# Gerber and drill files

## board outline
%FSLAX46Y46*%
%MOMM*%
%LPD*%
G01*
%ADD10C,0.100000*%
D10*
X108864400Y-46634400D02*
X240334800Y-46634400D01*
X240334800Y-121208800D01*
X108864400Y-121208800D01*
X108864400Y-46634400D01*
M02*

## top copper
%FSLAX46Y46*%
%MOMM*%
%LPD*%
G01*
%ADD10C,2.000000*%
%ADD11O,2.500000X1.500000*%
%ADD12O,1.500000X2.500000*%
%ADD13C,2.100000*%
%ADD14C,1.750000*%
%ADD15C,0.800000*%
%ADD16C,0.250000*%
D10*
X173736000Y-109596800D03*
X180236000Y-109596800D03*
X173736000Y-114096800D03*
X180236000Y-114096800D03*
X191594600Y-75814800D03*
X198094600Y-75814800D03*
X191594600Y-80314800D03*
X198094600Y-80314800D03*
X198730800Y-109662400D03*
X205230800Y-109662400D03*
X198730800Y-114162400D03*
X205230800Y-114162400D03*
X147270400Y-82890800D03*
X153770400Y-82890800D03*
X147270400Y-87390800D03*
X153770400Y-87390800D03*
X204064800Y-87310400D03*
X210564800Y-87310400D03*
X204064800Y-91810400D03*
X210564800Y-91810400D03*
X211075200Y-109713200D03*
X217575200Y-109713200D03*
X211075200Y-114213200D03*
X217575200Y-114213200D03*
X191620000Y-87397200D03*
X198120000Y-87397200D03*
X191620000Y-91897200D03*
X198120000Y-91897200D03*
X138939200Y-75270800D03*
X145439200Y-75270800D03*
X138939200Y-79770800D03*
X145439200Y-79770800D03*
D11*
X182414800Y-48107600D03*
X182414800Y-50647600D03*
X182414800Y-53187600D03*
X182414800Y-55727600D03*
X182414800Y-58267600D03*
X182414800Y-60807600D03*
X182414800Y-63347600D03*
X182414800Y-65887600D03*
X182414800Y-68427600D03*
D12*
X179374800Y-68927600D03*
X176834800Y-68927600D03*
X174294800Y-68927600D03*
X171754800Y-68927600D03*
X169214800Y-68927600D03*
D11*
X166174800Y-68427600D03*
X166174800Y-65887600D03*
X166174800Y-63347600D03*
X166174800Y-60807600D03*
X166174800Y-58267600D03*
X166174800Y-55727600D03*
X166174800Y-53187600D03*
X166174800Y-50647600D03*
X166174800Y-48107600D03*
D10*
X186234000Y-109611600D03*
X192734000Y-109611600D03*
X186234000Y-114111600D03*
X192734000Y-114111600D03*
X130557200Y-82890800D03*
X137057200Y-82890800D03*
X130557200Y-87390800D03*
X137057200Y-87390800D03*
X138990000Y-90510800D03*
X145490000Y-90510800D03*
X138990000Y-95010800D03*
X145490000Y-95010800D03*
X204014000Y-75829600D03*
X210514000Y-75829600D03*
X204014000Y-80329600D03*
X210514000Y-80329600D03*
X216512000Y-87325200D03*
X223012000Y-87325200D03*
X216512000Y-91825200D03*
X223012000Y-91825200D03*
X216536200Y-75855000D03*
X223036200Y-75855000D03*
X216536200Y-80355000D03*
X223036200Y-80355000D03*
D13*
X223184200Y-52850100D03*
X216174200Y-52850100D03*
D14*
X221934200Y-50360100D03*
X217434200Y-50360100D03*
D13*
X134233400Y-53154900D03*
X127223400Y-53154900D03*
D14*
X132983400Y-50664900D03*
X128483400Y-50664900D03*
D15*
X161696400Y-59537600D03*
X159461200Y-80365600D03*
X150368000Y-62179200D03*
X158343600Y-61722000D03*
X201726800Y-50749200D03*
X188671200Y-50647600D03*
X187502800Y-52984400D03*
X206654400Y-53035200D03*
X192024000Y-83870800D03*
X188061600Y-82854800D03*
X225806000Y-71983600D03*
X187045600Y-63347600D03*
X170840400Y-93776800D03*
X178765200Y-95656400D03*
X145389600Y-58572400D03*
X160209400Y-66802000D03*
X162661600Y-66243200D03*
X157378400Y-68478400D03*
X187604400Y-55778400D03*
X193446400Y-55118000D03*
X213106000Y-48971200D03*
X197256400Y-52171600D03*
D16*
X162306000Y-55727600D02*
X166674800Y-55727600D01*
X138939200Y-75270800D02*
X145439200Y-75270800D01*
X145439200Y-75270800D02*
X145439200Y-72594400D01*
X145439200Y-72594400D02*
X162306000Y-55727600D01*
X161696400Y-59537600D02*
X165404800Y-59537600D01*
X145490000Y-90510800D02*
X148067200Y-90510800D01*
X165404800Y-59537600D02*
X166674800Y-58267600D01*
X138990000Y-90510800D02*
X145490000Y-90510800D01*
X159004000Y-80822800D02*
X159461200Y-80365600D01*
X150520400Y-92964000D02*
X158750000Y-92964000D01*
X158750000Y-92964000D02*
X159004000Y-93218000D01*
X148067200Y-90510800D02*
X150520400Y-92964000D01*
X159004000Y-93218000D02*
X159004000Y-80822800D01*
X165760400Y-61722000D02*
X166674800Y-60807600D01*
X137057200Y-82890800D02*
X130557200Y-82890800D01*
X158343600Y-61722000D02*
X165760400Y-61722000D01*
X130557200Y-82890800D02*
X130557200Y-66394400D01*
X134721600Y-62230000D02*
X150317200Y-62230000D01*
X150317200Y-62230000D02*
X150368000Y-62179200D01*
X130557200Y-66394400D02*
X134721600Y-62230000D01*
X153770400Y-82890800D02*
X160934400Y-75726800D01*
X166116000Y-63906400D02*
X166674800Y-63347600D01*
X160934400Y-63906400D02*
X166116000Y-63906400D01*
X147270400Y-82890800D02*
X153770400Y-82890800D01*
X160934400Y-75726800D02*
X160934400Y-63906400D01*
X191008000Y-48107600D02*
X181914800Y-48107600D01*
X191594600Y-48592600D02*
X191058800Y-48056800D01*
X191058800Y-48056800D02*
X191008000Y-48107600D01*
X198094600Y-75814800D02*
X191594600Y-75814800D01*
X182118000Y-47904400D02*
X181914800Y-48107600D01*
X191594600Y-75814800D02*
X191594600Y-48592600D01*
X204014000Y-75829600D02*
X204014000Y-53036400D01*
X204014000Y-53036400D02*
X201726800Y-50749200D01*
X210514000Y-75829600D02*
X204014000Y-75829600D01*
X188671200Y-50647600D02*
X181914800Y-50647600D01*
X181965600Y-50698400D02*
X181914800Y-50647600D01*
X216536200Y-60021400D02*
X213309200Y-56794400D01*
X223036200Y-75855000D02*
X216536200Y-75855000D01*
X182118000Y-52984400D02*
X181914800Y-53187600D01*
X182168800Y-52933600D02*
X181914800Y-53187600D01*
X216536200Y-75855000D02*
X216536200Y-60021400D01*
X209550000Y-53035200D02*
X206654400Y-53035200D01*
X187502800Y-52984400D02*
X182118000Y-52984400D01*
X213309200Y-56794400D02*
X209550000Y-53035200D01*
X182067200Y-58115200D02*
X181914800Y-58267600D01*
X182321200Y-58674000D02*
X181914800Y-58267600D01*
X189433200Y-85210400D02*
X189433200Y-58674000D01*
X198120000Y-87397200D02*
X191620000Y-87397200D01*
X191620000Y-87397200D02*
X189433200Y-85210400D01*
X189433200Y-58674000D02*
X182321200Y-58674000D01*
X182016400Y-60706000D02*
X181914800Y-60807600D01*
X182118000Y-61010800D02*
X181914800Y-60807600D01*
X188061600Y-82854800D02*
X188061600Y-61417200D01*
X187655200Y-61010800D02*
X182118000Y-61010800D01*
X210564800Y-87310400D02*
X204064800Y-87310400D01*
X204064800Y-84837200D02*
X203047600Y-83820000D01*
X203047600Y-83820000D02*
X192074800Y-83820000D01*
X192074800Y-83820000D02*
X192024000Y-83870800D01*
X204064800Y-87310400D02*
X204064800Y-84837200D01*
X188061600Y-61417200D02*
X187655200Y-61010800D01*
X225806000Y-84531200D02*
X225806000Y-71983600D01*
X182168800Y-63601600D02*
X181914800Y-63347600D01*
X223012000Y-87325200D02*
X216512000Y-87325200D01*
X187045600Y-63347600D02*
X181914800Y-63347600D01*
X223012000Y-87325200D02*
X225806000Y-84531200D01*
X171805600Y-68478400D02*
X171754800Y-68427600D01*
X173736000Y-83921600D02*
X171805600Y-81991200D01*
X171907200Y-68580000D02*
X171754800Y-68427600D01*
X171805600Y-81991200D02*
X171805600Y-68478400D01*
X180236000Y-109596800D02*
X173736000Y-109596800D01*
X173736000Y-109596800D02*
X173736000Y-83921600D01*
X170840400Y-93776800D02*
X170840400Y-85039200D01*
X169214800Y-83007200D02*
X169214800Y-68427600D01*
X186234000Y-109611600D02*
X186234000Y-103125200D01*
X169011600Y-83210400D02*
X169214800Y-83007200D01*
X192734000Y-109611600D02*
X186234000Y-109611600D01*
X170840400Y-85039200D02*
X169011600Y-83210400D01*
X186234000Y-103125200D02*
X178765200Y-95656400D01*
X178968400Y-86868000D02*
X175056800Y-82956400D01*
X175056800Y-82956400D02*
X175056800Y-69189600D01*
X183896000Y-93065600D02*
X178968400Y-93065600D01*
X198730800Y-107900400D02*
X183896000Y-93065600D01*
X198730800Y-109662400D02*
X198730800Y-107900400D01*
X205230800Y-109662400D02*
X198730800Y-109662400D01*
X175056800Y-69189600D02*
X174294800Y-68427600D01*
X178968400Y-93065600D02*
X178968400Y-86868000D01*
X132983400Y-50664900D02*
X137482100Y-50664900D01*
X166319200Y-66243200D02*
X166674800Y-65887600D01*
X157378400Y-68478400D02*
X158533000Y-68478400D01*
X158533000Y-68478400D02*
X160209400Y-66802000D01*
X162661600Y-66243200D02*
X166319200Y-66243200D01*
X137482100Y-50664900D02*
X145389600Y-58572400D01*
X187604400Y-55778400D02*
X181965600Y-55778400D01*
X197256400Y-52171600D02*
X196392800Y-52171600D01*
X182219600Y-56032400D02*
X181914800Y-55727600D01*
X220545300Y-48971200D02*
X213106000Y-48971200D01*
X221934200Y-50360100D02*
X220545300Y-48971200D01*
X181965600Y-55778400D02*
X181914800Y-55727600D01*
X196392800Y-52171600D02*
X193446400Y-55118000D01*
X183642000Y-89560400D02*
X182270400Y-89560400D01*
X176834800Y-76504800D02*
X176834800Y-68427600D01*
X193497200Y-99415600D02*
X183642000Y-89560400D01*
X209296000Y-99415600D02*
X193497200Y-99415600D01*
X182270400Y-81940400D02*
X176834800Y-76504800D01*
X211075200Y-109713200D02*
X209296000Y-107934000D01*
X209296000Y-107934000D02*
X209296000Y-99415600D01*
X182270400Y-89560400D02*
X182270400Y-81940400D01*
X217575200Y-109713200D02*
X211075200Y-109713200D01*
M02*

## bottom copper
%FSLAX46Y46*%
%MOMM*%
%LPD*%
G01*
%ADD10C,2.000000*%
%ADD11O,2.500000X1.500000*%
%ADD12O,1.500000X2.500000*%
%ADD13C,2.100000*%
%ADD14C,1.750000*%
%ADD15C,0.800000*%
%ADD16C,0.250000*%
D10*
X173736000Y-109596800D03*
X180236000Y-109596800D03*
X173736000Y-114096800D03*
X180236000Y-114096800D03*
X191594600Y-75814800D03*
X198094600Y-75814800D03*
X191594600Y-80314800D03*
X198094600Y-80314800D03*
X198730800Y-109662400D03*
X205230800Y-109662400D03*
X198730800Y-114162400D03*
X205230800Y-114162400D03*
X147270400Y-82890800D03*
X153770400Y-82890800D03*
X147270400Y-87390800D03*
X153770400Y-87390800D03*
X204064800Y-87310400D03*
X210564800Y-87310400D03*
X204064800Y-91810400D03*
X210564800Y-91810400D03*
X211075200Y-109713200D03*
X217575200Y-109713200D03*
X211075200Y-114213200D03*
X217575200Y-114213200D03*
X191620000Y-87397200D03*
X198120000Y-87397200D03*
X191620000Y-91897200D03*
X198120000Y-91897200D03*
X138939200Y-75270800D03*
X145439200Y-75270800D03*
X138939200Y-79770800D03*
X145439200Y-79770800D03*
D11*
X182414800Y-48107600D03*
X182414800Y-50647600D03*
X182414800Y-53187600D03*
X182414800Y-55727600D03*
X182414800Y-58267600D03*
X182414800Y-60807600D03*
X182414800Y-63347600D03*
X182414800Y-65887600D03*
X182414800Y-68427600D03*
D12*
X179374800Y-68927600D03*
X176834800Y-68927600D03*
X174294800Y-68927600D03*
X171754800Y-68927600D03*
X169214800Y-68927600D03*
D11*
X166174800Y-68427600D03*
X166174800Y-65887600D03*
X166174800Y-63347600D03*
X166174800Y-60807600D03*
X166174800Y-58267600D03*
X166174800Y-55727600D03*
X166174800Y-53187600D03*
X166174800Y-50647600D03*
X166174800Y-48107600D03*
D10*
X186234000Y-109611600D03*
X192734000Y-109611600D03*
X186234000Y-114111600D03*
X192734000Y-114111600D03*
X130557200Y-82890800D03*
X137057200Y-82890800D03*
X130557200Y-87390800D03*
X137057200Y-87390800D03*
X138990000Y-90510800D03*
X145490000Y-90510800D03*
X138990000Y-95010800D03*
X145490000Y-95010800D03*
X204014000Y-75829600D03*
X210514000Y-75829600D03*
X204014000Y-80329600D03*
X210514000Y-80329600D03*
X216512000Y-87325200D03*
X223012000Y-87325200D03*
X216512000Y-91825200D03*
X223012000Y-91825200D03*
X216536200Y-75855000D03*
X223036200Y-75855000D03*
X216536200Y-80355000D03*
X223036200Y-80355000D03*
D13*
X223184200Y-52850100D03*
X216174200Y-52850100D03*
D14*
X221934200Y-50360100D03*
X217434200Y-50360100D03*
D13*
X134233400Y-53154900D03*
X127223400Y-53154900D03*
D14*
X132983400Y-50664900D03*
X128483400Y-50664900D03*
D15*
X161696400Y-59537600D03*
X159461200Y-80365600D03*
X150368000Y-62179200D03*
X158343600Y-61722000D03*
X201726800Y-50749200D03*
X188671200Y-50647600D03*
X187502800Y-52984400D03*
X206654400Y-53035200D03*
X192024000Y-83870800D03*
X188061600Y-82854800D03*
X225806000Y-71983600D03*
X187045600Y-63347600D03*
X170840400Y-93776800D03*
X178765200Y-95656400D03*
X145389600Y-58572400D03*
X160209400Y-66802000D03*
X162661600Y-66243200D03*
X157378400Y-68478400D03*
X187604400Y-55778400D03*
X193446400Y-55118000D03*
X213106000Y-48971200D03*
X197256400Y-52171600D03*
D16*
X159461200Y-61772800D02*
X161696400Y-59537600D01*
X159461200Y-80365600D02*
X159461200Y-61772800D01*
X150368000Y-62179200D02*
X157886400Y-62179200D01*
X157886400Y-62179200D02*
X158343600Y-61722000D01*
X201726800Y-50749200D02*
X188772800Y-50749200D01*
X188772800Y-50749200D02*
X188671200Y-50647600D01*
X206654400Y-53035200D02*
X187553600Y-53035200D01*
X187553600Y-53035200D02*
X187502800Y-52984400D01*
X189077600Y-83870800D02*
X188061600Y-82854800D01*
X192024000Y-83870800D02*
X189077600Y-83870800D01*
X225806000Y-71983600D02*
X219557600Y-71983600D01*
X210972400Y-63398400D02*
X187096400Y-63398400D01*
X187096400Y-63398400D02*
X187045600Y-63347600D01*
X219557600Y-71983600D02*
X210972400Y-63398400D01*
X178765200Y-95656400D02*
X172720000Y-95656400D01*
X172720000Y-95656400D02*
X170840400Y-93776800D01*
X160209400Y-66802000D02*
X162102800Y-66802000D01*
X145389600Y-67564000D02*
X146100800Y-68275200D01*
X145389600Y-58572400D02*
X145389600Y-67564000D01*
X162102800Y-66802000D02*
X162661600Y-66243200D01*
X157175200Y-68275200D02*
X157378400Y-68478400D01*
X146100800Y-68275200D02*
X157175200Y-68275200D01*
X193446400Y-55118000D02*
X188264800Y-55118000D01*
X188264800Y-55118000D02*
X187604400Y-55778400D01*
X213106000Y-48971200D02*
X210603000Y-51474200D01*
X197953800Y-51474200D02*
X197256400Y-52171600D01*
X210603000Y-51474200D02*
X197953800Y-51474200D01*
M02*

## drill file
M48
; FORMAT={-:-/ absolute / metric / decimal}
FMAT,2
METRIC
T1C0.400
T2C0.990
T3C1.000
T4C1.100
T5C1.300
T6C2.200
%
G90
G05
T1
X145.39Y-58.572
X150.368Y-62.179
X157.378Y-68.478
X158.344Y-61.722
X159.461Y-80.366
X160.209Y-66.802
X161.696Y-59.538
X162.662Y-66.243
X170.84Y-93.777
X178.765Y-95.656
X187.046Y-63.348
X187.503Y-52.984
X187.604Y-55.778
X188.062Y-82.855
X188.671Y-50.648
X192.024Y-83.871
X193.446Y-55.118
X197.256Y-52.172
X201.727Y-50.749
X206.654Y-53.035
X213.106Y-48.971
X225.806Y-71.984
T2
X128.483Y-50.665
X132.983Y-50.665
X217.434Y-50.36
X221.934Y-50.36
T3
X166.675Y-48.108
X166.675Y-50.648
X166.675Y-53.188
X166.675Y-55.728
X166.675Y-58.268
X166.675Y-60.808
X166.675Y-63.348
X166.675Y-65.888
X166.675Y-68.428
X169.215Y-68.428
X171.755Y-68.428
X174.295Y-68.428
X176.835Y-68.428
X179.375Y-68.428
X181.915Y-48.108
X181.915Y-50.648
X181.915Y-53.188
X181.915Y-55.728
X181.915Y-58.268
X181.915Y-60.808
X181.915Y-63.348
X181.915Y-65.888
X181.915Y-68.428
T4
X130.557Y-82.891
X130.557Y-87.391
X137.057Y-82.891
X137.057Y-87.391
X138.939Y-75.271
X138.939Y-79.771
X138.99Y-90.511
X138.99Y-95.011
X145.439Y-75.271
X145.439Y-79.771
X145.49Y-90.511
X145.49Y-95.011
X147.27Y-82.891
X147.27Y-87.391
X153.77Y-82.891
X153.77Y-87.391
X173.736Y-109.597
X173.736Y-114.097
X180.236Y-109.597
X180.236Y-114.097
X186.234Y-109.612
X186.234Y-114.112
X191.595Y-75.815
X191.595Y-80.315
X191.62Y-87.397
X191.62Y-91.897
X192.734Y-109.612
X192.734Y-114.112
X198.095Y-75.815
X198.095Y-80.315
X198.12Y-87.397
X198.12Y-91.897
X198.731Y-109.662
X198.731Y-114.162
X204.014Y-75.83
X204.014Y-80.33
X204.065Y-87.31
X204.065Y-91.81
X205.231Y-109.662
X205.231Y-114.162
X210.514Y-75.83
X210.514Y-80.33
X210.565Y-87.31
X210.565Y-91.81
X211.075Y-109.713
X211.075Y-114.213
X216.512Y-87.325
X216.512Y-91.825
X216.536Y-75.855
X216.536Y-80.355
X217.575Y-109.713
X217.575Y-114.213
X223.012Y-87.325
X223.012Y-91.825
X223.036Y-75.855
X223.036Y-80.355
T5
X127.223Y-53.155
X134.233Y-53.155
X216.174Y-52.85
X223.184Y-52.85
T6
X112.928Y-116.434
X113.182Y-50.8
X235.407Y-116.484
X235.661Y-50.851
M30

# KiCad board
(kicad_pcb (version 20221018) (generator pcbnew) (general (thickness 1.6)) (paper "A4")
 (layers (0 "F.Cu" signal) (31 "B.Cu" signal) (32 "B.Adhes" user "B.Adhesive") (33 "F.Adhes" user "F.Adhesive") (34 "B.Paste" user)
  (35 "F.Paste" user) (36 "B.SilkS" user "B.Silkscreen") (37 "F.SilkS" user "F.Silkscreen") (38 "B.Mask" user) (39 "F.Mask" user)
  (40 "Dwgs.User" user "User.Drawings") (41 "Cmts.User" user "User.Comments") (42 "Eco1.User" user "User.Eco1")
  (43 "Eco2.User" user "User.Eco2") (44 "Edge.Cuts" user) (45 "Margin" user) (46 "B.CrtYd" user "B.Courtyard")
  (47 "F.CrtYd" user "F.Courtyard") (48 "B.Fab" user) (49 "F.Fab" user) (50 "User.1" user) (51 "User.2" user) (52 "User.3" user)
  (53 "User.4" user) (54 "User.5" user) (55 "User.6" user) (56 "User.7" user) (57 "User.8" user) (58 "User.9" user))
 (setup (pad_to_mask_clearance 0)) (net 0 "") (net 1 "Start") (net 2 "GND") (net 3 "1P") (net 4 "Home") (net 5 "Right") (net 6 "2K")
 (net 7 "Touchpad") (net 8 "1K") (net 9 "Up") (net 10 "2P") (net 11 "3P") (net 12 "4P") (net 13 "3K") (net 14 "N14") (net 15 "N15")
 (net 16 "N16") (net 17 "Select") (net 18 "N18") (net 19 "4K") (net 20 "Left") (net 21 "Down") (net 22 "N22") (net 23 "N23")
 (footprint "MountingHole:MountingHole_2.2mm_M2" (layer "F.Cu") (at 112.9284 116.4336)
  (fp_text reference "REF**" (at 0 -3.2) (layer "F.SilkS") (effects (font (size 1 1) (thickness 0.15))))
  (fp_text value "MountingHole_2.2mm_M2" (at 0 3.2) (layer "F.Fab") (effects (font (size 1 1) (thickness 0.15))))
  (pad "" np_thru_hole circle (at 0 0) (size 2.2 2.2) (drill 2.2) (layers "F&B.Cu" "*.Mask")))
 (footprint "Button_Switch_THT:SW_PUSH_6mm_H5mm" (layer "F.Cu") (at 173.736 109.5968)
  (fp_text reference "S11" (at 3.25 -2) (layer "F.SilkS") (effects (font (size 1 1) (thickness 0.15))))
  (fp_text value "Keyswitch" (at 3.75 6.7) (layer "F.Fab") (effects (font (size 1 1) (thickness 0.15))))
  (pad "1" thru_hole circle (at 0 0 90) (size 2 2) (drill 1.1) (layers "*.Cu" "*.Mask") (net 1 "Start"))
  (pad "1" thru_hole circle (at 6.5 0 90) (size 2 2) (drill 1.1) (layers "*.Cu" "*.Mask") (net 1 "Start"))
  (pad "2" thru_hole circle (at 0 4.5 90) (size 2 2) (drill 1.1) (layers "*.Cu" "*.Mask") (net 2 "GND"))
  (pad "2" thru_hole circle (at 6.5 4.5 90) (size 2 2) (drill 1.1) (layers "*.Cu" "*.Mask") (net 2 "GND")))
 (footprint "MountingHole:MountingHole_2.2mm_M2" (layer "F.Cu") (at 113.1824 50.8)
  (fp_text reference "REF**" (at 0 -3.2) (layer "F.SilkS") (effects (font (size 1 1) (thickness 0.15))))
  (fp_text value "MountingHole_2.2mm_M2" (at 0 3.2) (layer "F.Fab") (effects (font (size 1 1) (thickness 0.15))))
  (pad "" np_thru_hole circle (at 0 0) (size 2.2 2.2) (drill 2.2) (layers "F&B.Cu" "*.Mask")))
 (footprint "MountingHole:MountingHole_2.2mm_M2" (layer "F.Cu") (at 235.4072 116.4844)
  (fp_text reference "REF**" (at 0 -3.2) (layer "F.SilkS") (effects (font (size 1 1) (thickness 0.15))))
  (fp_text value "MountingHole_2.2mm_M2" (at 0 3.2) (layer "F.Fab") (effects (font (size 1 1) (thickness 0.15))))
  (pad "" np_thru_hole circle (at 0 0) (size 2.2 2.2) (drill 2.2) (layers "F&B.Cu" "*.Mask")))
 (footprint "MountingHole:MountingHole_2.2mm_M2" (layer "F.Cu") (at 235.6612 50.8508)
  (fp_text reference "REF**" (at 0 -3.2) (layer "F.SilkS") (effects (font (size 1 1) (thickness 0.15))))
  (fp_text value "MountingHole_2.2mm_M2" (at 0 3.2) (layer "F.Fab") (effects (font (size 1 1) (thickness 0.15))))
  (pad "" np_thru_hole circle (at 0 0) (size 2.2 2.2) (drill 2.2) (layers "*.Cu" "*.Mask")))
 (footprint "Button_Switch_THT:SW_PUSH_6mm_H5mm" (layer "F.Cu") (at 191.5946 75.8148)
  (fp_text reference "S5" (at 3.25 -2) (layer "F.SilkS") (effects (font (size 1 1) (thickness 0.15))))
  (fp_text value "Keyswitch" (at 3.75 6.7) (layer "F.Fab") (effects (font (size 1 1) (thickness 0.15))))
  (pad "1" thru_hole circle (at 0 0 90) (size 2 2) (drill 1.1) (layers "*.Cu" "*.Mask") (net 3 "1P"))
  (pad "1" thru_hole circle (at 6.5 0 90) (size 2 2) (drill 1.1) (layers "*.Cu" "*.Mask") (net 3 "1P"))
  (pad "2" thru_hole circle (at 0 4.5 90) (size 2 2) (drill 1.1) (layers "*.Cu" "*.Mask") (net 2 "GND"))
  (pad "2" thru_hole circle (at 6.5 4.5 90) (size 2 2) (drill 1.1) (layers "*.Cu" "*.Mask") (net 2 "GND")))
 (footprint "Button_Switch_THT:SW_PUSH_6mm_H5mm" (layer "F.Cu") (at 198.7308 109.6624)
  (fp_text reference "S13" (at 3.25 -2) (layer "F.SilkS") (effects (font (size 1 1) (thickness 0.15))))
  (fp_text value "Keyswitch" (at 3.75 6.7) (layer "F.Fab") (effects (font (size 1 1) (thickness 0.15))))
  (pad "1" thru_hole circle (at 0 0 90) (size 2 2) (drill 1.1) (layers "*.Cu" "*.Mask") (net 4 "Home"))
  (pad "1" thru_hole circle (at 6.5 0 90) (size 2 2) (drill 1.1) (layers "*.Cu" "*.Mask") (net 4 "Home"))
  (pad "2" thru_hole circle (at 0 4.5 90) (size 2 2) (drill 1.1) (layers "*.Cu" "*.Mask") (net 2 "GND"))
  (pad "2" thru_hole circle (at 6.5 4.5 90) (size 2 2) (drill 1.1) (layers "*.Cu" "*.Mask") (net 2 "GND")))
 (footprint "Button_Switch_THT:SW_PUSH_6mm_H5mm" (layer "F.Cu") (at 147.2704 82.8908)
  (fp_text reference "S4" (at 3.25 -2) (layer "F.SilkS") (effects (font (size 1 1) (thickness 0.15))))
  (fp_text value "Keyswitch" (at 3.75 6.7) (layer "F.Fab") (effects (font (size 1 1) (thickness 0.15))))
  (pad "1" thru_hole circle (at 0 0 90) (size 2 2) (drill 1.1) (layers "*.Cu" "*.Mask") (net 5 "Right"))
  (pad "1" thru_hole circle (at 6.5 0 90) (size 2 2) (drill 1.1) (layers "*.Cu" "*.Mask") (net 5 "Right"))
  (pad "2" thru_hole circle (at 0 4.5 90) (size 2 2) (drill 1.1) (layers "*.Cu" "*.Mask") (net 2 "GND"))
  (pad "2" thru_hole circle (at 6.5 4.5 90) (size 2 2) (drill 1.1) (layers "*.Cu" "*.Mask") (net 2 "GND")))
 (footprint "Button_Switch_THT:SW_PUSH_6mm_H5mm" (layer "F.Cu") (at 204.0648 87.3104)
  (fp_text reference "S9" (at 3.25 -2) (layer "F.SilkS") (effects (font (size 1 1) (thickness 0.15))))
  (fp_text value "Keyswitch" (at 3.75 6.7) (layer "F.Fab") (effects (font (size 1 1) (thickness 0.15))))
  (pad "1" thru_hole circle (at 0 0 90) (size 2 2) (drill 1.1) (layers "*.Cu" "*.Mask") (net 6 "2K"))
  (pad "1" thru_hole circle (at 6.5 0 90) (size 2 2) (drill 1.1) (layers "*.Cu" "*.Mask") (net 6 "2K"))
  (pad "2" thru_hole circle (at 0 4.5 90) (size 2 2) (drill 1.1) (layers "*.Cu" "*.Mask") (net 2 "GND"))
  (pad "2" thru_hole circle (at 6.5 4.5 90) (size 2 2) (drill 1.1) (layers "*.Cu" "*.Mask") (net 2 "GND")))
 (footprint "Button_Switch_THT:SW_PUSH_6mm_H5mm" (layer "F.Cu") (at 211.0752 109.7132)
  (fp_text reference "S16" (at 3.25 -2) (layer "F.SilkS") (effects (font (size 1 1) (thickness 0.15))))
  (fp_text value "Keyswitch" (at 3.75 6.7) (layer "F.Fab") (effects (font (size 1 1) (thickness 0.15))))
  (pad "1" thru_hole circle (at 0 0 90) (size 2 2) (drill 1.1) (layers "*.Cu" "*.Mask") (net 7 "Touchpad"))
  (pad "1" thru_hole circle (at 6.5 0 90) (size 2 2) (drill 1.1) (layers "*.Cu" "*.Mask") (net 7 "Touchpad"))
  (pad "2" thru_hole circle (at 0 4.5 90) (size 2 2) (drill 1.1) (layers "*.Cu" "*.Mask") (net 2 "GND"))
  (pad "2" thru_hole circle (at 6.5 4.5 90) (size 2 2) (drill 1.1) (layers "*.Cu" "*.Mask") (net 2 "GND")))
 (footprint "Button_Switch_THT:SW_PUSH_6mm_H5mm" (layer "F.Cu") (at 191.62 87.3972)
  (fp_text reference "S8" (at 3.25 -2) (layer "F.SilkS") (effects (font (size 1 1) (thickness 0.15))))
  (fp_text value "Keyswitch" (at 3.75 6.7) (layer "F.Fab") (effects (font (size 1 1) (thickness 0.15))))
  (pad "1" thru_hole circle (at 0 0 90) (size 2 2) (drill 1.1) (layers "*.Cu" "*.Mask") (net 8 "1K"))
  (pad "1" thru_hole circle (at 6.5 0 90) (size 2 2) (drill 1.1) (layers "*.Cu" "*.Mask") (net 8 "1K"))
  (pad "2" thru_hole circle (at 0 4.5 90) (size 2 2) (drill 1.1) (layers "*.Cu" "*.Mask") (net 2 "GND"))
  (pad "2" thru_hole circle (at 6.5 4.5 90) (size 2 2) (drill 1.1) (layers "*.Cu" "*.Mask") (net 2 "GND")))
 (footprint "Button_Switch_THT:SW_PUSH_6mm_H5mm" (layer "F.Cu") (at 138.9392 75.2708)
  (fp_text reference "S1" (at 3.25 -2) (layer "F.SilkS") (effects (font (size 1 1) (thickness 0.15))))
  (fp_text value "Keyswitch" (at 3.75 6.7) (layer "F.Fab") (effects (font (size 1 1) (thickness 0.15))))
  (pad "1" thru_hole circle (at 0 0 90) (size 2 2) (drill 1.1) (layers "*.Cu" "*.Mask") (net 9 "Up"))
  (pad "1" thru_hole circle (at 6.5 0 90) (size 2 2) (drill 1.1) (layers "*.Cu" "*.Mask") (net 9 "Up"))
  (pad "2" thru_hole circle (at 0 4.5 90) (size 2 2) (drill 1.1) (layers "*.Cu" "*.Mask") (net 2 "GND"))
  (pad "2" thru_hole circle (at 6.5 4.5 90) (size 2 2) (drill 1.1) (layers "*.Cu" "*.Mask") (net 2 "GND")))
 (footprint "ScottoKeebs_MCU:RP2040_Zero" (layer "F.Cu") (at 174.2948 58.2676)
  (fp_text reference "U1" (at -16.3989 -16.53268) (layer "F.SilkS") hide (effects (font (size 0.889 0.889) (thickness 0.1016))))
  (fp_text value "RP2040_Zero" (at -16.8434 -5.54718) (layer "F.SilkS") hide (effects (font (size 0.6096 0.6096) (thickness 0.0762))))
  (pad "1" thru_hole oval (at 7.62 -10.16 180) (size 2.5 1.5) (drill 1 (offset -0.5 0)) (layers "*.Cu" "*.Mask") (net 3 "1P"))
  (pad "2" thru_hole oval (at 7.62 -7.62 180) (size 2.5 1.5) (drill 1 (offset -0.5 0)) (layers "*.Cu" "*.Mask") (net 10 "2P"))
  (pad "3" thru_hole oval (at 7.62 -5.08 180) (size 2.5 1.5) (drill 1 (offset -0.5 0)) (layers "*.Cu" "*.Mask") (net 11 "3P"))
  (pad "4" thru_hole oval (at 7.62 -2.54 180) (size 2.5 1.5) (drill 1 (offset -0.5 0)) (layers "*.Cu" "*.Mask") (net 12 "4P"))
  (pad "5" thru_hole oval (at 7.62 0 180) (size 2.5 1.5) (drill 1 (offset -0.5 0)) (layers "*.Cu" "*.Mask") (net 8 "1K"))
  (pad "6" thru_hole oval (at 7.62 2.54 180) (size 2.5 1.5) (drill 1 (offset -0.5 0)) (layers "*.Cu" "*.Mask") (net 6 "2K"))
  (pad "7" thru_hole oval (at 7.62 5.08 180) (size 2.5 1.5) (drill 1 (offset -0.5 0)) (layers "*.Cu" "*.Mask") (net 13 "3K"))
  (pad "8" thru_hole oval (at 7.62 7.62 180) (size 2.5 1.5) (drill 1 (offset -0.5 0)) (layers "*.Cu" "*.Mask") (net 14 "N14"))
  (pad "9" thru_hole oval (at 7.62 10.16 180) (size 2.5 1.5) (drill 1 (offset -0.5 0)) (layers "*.Cu" "*.Mask") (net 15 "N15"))
  (pad "10" thru_hole oval (at 5.08 10.16 90) (size 2.5 1.5) (drill 1 (offset -0.5 0)) (layers "*.Cu" "*.Mask") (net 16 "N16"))
  (pad "11" thru_hole oval (at 2.54 10.16 90) (size 2.5 1.5) (drill 1 (offset -0.5 0)) (layers "*.Cu" "*.Mask") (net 7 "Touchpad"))
  (pad "12" thru_hole oval (at 0 10.16 90) (size 2.5 1.5) (drill 1 (offset -0.5 0)) (layers "*.Cu" "*.Mask") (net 4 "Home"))
  (pad "13" thru_hole oval (at -2.54 10.16 90) (size 2.5 1.5) (drill 1 (offset -0.5 0)) (layers "*.Cu" "*.Mask") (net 1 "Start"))
  (pad "14" thru_hole oval (at -5.08 10.16 90) (size 2.5 1.5) (drill 1 (offset -0.5 0)) (layers "*.Cu" "*.Mask") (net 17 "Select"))
  (pad "15" thru_hole oval (at -7.62 10.16) (size 2.5 1.5) (drill 1 (offset -0.5 0)) (layers "*.Cu" "*.Mask") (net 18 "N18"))
  (pad "16" thru_hole oval (at -7.62 7.62) (size 2.5 1.5) (drill 1 (offset -0.5 0)) (layers "*.Cu" "*.Mask") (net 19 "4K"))
  (pad "17" thru_hole oval (at -7.62 5.08) (size 2.5 1.5) (drill 1 (offset -0.5 0)) (layers "*.Cu" "*.Mask") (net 5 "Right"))
  (pad "18" thru_hole oval (at -7.62 2.54) (size 2.5 1.5) (drill 1 (offset -0.5 0)) (layers "*.Cu" "*.Mask") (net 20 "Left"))
  (pad "19" thru_hole oval (at -7.62 0) (size 2.5 1.5) (drill 1 (offset -0.5 0)) (layers "*.Cu" "*.Mask") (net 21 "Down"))
  (pad "20" thru_hole oval (at -7.62 -2.54) (size 2.5 1.5) (drill 1 (offset -0.5 0)) (layers "*.Cu" "*.Mask") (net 9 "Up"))
  (pad "21" thru_hole oval (at -7.62 -5.08) (size 2.5 1.5) (drill 1 (offset -0.5 0)) (layers "*.Cu" "*.Mask") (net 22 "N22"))
  (pad "22" thru_hole oval (at -7.62 -7.62) (size 2.5 1.5) (drill 1 (offset -0.5 0)) (layers "*.Cu" "*.Mask") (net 2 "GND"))
  (pad "23" thru_hole oval (at -7.62 -10.16) (size 2.5 1.5) (drill 1 (offset -0.5 0)) (layers "*.Cu" "*.Mask") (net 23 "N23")))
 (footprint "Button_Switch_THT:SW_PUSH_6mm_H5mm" (layer "F.Cu") (at 186.234 109.6116)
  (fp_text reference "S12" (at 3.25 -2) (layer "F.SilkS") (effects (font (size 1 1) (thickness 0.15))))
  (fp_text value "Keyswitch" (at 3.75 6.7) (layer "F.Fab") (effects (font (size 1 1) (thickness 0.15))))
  (pad "1" thru_hole circle (at 0 0 90) (size 2 2) (drill 1.1) (layers "*.Cu" "*.Mask") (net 17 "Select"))
  (pad "1" thru_hole circle (at 6.5 0 90) (size 2 2) (drill 1.1) (layers "*.Cu" "*.Mask") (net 17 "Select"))
  (pad "2" thru_hole circle (at 0 4.5 90) (size 2 2) (drill 1.1) (layers "*.Cu" "*.Mask") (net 2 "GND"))
  (pad "2" thru_hole circle (at 6.5 4.5 90) (size 2 2) (drill 1.1) (layers "*.Cu" "*.Mask") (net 2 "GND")))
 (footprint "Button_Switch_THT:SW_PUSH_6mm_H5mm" (layer "F.Cu") (at 130.5572 82.8908)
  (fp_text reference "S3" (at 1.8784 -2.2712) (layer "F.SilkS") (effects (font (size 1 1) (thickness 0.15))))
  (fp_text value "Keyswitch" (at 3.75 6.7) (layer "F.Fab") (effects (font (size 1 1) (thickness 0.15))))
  (pad "1" thru_hole circle (at 0 0 90) (size 2 2) (drill 1.1) (layers "*.Cu" "*.Mask") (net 20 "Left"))
  (pad "1" thru_hole circle (at 6.5 0 90) (size 2 2) (drill 1.1) (layers "*.Cu" "*.Mask") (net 20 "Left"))
  (pad "2" thru_hole circle (at 0 4.5 90) (size 2 2) (drill 1.1) (layers "*.Cu" "*.Mask") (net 2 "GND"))
  (pad "2" thru_hole circle (at 6.5 4.5 90) (size 2 2) (drill 1.1) (layers "*.Cu" "*.Mask") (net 2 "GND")))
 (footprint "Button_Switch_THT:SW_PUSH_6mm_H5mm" (layer "F.Cu") (at 138.99 90.5108)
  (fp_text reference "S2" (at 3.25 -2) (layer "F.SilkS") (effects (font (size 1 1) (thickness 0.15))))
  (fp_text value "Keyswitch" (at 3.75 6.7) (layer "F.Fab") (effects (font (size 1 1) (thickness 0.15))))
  (pad "1" thru_hole circle (at 0 0 90) (size 2 2) (drill 1.1) (layers "*.Cu" "*.Mask") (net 21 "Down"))
  (pad "1" thru_hole circle (at 6.5 0 90) (size 2 2) (drill 1.1) (layers "*.Cu" "*.Mask") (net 21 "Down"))
  (pad "2" thru_hole circle (at 0 4.5 90) (size 2 2) (drill 1.1) (layers "*.Cu" "*.Mask") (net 2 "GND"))
  (pad "2" thru_hole circle (at 6.5 4.5 90) (size 2 2) (drill 1.1) (layers "*.Cu" "*.Mask") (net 2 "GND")))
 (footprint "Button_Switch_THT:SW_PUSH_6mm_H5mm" (layer "F.Cu") (at 204.014 75.8296)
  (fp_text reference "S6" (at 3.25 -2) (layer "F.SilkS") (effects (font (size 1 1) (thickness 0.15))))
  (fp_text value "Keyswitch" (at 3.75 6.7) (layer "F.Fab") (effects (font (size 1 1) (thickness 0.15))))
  (pad "1" thru_hole circle (at 0 0 90) (size 2 2) (drill 1.1) (layers "*.Cu" "*.Mask") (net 10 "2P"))
  (pad "1" thru_hole circle (at 6.5 0 90) (size 2 2) (drill 1.1) (layers "*.Cu" "*.Mask") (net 10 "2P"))
  (pad "2" thru_hole circle (at 0 4.5 90) (size 2 2) (drill 1.1) (layers "*.Cu" "*.Mask") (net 2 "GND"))
  (pad "2" thru_hole circle (at 6.5 4.5 90) (size 2 2) (drill 1.1) (layers "*.Cu" "*.Mask") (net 2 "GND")))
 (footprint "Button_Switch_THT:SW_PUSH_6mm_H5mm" (layer "F.Cu") (at 216.512 87.3252)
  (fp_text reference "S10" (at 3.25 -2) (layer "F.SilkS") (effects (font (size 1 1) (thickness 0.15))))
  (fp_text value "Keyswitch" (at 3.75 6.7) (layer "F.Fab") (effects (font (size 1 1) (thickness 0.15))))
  (pad "1" thru_hole circle (at 0 0 90) (size 2 2) (drill 1.1) (layers "*.Cu" "*.Mask") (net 13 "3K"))
  (pad "1" thru_hole circle (at 6.5 0 90) (size 2 2) (drill 1.1) (layers "*.Cu" "*.Mask") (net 13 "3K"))
  (pad "2" thru_hole circle (at 0 4.5 90) (size 2 2) (drill 1.1) (layers "*.Cu" "*.Mask") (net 2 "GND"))
  (pad "2" thru_hole circle (at 6.5 4.5 90) (size 2 2) (drill 1.1) (layers "*.Cu" "*.Mask") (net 2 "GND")))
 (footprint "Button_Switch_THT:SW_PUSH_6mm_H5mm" (layer "F.Cu") (at 216.5362 75.855)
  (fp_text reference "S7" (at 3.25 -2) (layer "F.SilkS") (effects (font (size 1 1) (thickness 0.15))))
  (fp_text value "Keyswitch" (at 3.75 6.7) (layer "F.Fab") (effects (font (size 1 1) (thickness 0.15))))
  (pad "1" thru_hole circle (at 0 0 90) (size 2 2) (drill 1.1) (layers "*.Cu" "*.Mask") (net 11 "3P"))
  (pad "1" thru_hole circle (at 6.5 0 90) (size 2 2) (drill 1.1) (layers "*.Cu" "*.Mask") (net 11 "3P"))
  (pad "2" thru_hole circle (at 0 4.5 90) (size 2 2) (drill 1.1) (layers "*.Cu" "*.Mask") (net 2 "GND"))
  (pad "2" thru_hole circle (at 6.5 4.5 90) (size 2 2) (drill 1.1) (layers "*.Cu" "*.Mask") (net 2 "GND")))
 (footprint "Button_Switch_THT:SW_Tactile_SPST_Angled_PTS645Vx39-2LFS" (layer "B.Cu") (at 221.9342 50.3601 180)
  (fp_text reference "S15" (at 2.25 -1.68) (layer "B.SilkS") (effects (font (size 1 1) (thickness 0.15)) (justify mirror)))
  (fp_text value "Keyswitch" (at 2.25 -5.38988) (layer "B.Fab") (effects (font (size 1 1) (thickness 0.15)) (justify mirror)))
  (pad "" thru_hole circle (at -1.25 -2.49 180) (size 2.1 2.1) (drill 1.3) (layers "*.Cu" "*.Mask"))
  (pad "" thru_hole circle (at 5.76 -2.49 180) (size 2.1 2.1) (drill 1.3) (layers "*.Cu" "*.Mask"))
  (pad "1" thru_hole circle (at 0 0 180) (size 1.75 1.75) (drill 0.99) (layers "*.Cu" "*.Mask") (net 12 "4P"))
  (pad "2" thru_hole circle (at 4.5 0 180) (size 1.75 1.75) (drill 0.99) (layers "*.Cu" "*.Mask") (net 2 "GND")))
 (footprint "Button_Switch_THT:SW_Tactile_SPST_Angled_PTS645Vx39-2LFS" (layer "B.Cu") (at 132.9834 50.6649 180)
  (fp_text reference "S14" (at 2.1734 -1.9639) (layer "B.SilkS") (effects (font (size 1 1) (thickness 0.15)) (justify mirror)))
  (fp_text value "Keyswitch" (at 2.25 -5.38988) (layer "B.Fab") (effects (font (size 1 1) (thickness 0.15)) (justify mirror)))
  (pad "" thru_hole circle (at -1.25 -2.49 180) (size 2.1 2.1) (drill 1.3) (layers "*.Cu" "*.Mask"))
  (pad "" thru_hole circle (at 5.76 -2.49 180) (size 2.1 2.1) (drill 1.3) (layers "*.Cu" "*.Mask"))
  (pad "1" thru_hole circle (at 0 0 180) (size 1.75 1.75) (drill 0.99) (layers "*.Cu" "*.Mask") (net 19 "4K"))
  (pad "2" thru_hole circle (at 4.5 0 180) (size 1.75 1.75) (drill 0.99) (layers "*.Cu" "*.Mask") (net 2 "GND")))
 (gr_rect (start 108.8644 46.6344) (end 240.3348 121.2088) (stroke (width 0.1) (type default)) (fill none) (layer "Edge.Cuts"))
 (segment (start 162.306 55.7276) (end 166.6748 55.7276) (width 0.25) (layer "F.Cu") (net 9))
 (segment (start 138.9392 75.2708) (end 145.4392 75.2708) (width 0.25) (layer "F.Cu") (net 9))
 (segment (start 145.4392 75.2708) (end 145.4392 72.5944) (width 0.25) (layer "F.Cu") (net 9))
 (segment (start 145.4392 72.5944) (end 162.306 55.7276) (width 0.25) (layer "F.Cu") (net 9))
 (segment (start 161.6964 59.5376) (end 165.4048 59.5376) (width 0.25) (layer "F.Cu") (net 21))
 (segment (start 145.49 90.5108) (end 148.0672 90.5108) (width 0.25) (layer "F.Cu") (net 21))
 (segment (start 165.4048 59.5376) (end 166.6748 58.2676) (width 0.25) (layer "F.Cu") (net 21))
 (segment (start 138.99 90.5108) (end 145.49 90.5108) (width 0.25) (layer "F.Cu") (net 21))
 (segment (start 159.004 80.8228) (end 159.4612 80.3656) (width 0.25) (layer "F.Cu") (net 21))
 (segment (start 150.5204 92.964) (end 158.75 92.964) (width 0.25) (layer "F.Cu") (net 21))
 (segment (start 158.75 92.964) (end 159.004 93.218) (width 0.25) (layer "F.Cu") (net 21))
 (segment (start 148.0672 90.5108) (end 150.5204 92.964) (width 0.25) (layer "F.Cu") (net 21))
 (segment (start 159.004 93.218) (end 159.004 80.8228) (width 0.25) (layer "F.Cu") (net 21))
 (via (at 161.6964 59.5376) (size 0.8) (drill 0.4) (layers "F.Cu" "B.Cu") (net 21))
 (via (at 159.4612 80.3656) (size 0.8) (drill 0.4) (layers "F.Cu" "B.Cu") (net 21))
 (segment (start 159.4612 61.7728) (end 161.6964 59.5376) (width 0.25) (layer "B.Cu") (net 21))
 (segment (start 159.4612 80.3656) (end 159.4612 61.7728) (width 0.25) (layer "B.Cu") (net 21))
 (segment (start 165.7604 61.722) (end 166.6748 60.8076) (width 0.25) (layer "F.Cu") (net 20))
 (segment (start 137.0572 82.8908) (end 130.5572 82.8908) (width 0.25) (layer "F.Cu") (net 20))
 (segment (start 158.3436 61.722) (end 165.7604 61.722) (width 0.25) (layer "F.Cu") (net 20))
 (segment (start 130.5572 82.8908) (end 130.5572 66.3944) (width 0.25) (layer "F.Cu") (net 20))
 (segment (start 134.7216 62.23) (end 150.3172 62.23) (width 0.25) (layer "F.Cu") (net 20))
 (segment (start 150.3172 62.23) (end 150.368 62.1792) (width 0.25) (layer "F.Cu") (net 20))
 (segment (start 130.5572 66.3944) (end 134.7216 62.23) (width 0.25) (layer "F.Cu") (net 20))
 (via (at 150.368 62.1792) (size 0.8) (drill 0.4) (layers "F.Cu" "B.Cu") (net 20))
 (via (at 158.3436 61.722) (size 0.8) (drill 0.4) (layers "F.Cu" "B.Cu") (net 20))
 (segment (start 150.368 62.1792) (end 157.8864 62.1792) (width 0.25) (layer "B.Cu") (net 20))
 (segment (start 157.8864 62.1792) (end 158.3436 61.722) (width 0.25) (layer "B.Cu") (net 20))
 (segment (start 153.7704 82.8908) (end 160.9344 75.7268) (width 0.25) (layer "F.Cu") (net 5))
 (segment (start 166.116 63.9064) (end 166.6748 63.3476) (width 0.25) (layer "F.Cu") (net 5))
 (segment (start 160.9344 63.9064) (end 166.116 63.9064) (width 0.25) (layer "F.Cu") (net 5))
 (segment (start 147.2704 82.8908) (end 153.7704 82.8908) (width 0.25) (layer "F.Cu") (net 5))
 (segment (start 160.9344 75.7268) (end 160.9344 63.9064) (width 0.25) (layer "F.Cu") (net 5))
 (segment (start 191.008 48.1076) (end 181.9148 48.1076) (width 0.25) (layer "F.Cu") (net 3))
 (segment (start 191.5946 48.5926) (end 191.0588 48.0568) (width 0.25) (layer "F.Cu") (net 3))
 (segment (start 191.0588 48.0568) (end 191.008 48.1076) (width 0.25) (layer "F.Cu") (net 3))
 (segment (start 198.0946 75.8148) (end 191.5946 75.8148) (width 0.25) (layer "F.Cu") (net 3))
 (segment (start 182.118 47.9044) (end 181.9148 48.1076) (width 0.25) (layer "F.Cu") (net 3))
 (segment (start 191.5946 75.8148) (end 191.5946 48.5926) (width 0.25) (layer "F.Cu") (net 3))
 (segment (start 204.014 75.8296) (end 204.014 53.0364) (width 0.25) (layer "F.Cu") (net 10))
 (segment (start 204.014 53.0364) (end 201.7268 50.7492) (width 0.25) (layer "F.Cu") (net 10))
 (segment (start 210.514 75.8296) (end 204.014 75.8296) (width 0.25) (layer "F.Cu") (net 10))
 (segment (start 188.6712 50.6476) (end 181.9148 50.6476) (width 0.25) (layer "F.Cu") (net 10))
 (segment (start 181.9656 50.6984) (end 181.9148 50.6476) (width 0.25) (layer "F.Cu") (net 10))
 (via (at 201.7268 50.7492) (size 0.8) (drill 0.4) (layers "F.Cu" "B.Cu") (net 10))
 (via (at 188.6712 50.6476) (size 0.8) (drill 0.4) (layers "F.Cu" "B.Cu") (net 10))
 (segment (start 201.7268 50.7492) (end 188.7728 50.7492) (width 0.25) (layer "B.Cu") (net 10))
 (segment (start 188.7728 50.7492) (end 188.6712 50.6476) (width 0.25) (layer "B.Cu") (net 10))
 (segment (start 216.5362 60.0214) (end 213.3092 56.7944) (width 0.25) (layer "F.Cu") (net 11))
 (segment (start 223.0362 75.855) (end 216.5362 75.855) (width 0.25) (layer "F.Cu") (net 11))
 (segment (start 182.118 52.9844) (end 181.9148 53.1876) (width 0.25) (layer "F.Cu") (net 11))
 (segment (start 182.1688 52.9336) (end 181.9148 53.1876) (width 0.25) (layer "F.Cu") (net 11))
 (segment (start 216.5362 75.855) (end 216.5362 60.0214) (width 0.25) (layer "F.Cu") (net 11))
 (segment (start 209.55 53.0352) (end 206.6544 53.0352) (width 0.25) (layer "F.Cu") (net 11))
 (segment (start 187.5028 52.9844) (end 182.118 52.9844) (width 0.25) (layer "F.Cu") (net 11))
 (segment (start 213.3092 56.7944) (end 209.55 53.0352) (width 0.25) (layer "F.Cu") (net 11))
 (via (at 187.5028 52.9844) (size 0.8) (drill 0.4) (layers "F.Cu" "B.Cu") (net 11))
 (via (at 206.6544 53.0352) (size 0.8) (drill 0.4) (layers "F.Cu" "B.Cu") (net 11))
 (segment (start 206.6544 53.0352) (end 187.5536 53.0352) (width 0.25) (layer "B.Cu") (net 11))
 (segment (start 187.5536 53.0352) (end 187.5028 52.9844) (width 0.25) (layer "B.Cu") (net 11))
 (segment (start 182.0672 58.1152) (end 181.9148 58.2676) (width 0.25) (layer "F.Cu") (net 8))
 (segment (start 182.3212 58.674) (end 181.9148 58.2676) (width 0.25) (layer "F.Cu") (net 8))
 (segment (start 189.4332 85.2104) (end 189.4332 58.674) (width 0.25) (layer "F.Cu") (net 8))
 (segment (start 198.12 87.3972) (end 191.62 87.3972) (width 0.25) (layer "F.Cu") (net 8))
 (segment (start 191.62 87.3972) (end 189.4332 85.2104) (width 0.25) (layer "F.Cu") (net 8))
 (segment (start 189.4332 58.674) (end 182.3212 58.674) (width 0.25) (layer "F.Cu") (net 8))
 (segment (start 182.0164 60.706) (end 181.9148 60.8076) (width 0.25) (layer "F.Cu") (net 6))
 (segment (start 182.118 61.0108) (end 181.9148 60.8076) (width 0.25) (layer "F.Cu") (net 6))
 (segment (start 188.0616 82.8548) (end 188.0616 61.4172) (width 0.25) (layer "F.Cu") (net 6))
 (segment (start 187.6552 61.0108) (end 182.118 61.0108) (width 0.25) (layer "F.Cu") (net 6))
 (segment (start 210.5648 87.3104) (end 204.0648 87.3104) (width 0.25) (layer "F.Cu") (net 6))
 (segment (start 204.0648 84.8372) (end 203.0476 83.82) (width 0.25) (layer "F.Cu") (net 6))
 (segment (start 203.0476 83.82) (end 192.0748 83.82) (width 0.25) (layer "F.Cu") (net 6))
 (segment (start 192.0748 83.82) (end 192.024 83.8708) (width 0.25) (layer "F.Cu") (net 6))
 (segment (start 204.0648 87.3104) (end 204.0648 84.8372) (width 0.25) (layer "F.Cu") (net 6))
 (segment (start 188.0616 61.4172) (end 187.6552 61.0108) (width 0.25) (layer "F.Cu") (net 6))
 (via (at 192.024 83.8708) (size 0.8) (drill 0.4) (layers "F.Cu" "B.Cu") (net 6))
 (via (at 188.0616 82.8548) (size 0.8) (drill 0.4) (layers "F.Cu" "B.Cu") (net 6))
 (segment (start 189.0776 83.8708) (end 188.0616 82.8548) (width 0.25) (layer "B.Cu") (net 6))
 (segment (start 192.024 83.8708) (end 189.0776 83.8708) (width 0.25) (layer "B.Cu") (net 6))
 (segment (start 225.806 84.5312) (end 225.806 71.9836) (width 0.25) (layer "F.Cu") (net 13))
 (segment (start 182.1688 63.6016) (end 181.9148 63.3476) (width 0.25) (layer "F.Cu") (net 13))
 (segment (start 223.012 87.3252) (end 216.512 87.3252) (width 0.25) (layer "F.Cu") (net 13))
 (segment (start 187.0456 63.3476) (end 181.9148 63.3476) (width 0.25) (layer "F.Cu") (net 13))
 (segment (start 223.012 87.3252) (end 225.806 84.5312) (width 0.25) (layer "F.Cu") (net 13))
 (via (at 225.806 71.9836) (size 0.8) (drill 0.4) (layers "F.Cu" "B.Cu") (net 13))
 (via (at 187.0456 63.3476) (size 0.8) (drill 0.4) (layers "F.Cu" "B.Cu") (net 13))
 (segment (start 225.806 71.9836) (end 219.5576 71.9836) (width 0.25) (layer "B.Cu") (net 13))
 (segment (start 210.9724 63.3984) (end 187.0964 63.3984) (width 0.25) (layer "B.Cu") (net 13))
 (segment (start 187.0964 63.3984) (end 187.0456 63.3476) (width 0.25) (layer "B.Cu") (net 13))
 (segment (start 219.5576 71.9836) (end 210.9724 63.3984) (width 0.25) (layer "B.Cu") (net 13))
 (segment (start 171.8056 68.4784) (end 171.7548 68.4276) (width 0.25) (layer "F.Cu") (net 1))
 (segment (start 173.736 83.9216) (end 171.8056 81.9912) (width 0.25) (layer "F.Cu") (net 1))
 (segment (start 171.9072 68.58) (end 171.7548 68.4276) (width 0.25) (layer "F.Cu") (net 1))
 (segment (start 171.8056 81.9912) (end 171.8056 68.4784) (width 0.25) (layer "F.Cu") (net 1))
 (segment (start 180.236 109.5968) (end 173.736 109.5968) (width 0.25) (layer "F.Cu") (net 1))
 (segment (start 173.736 109.5968) (end 173.736 83.9216) (width 0.25) (layer "F.Cu") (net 1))
 (segment (start 170.8404 93.7768) (end 170.8404 85.0392) (width 0.25) (layer "F.Cu") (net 17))
 (segment (start 169.2148 83.0072) (end 169.2148 68.4276) (width 0.25) (layer "F.Cu") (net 17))
 (segment (start 186.234 109.6116) (end 186.234 103.1252) (width 0.25) (layer "F.Cu") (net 17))
 (segment (start 169.0116 83.2104) (end 169.2148 83.0072) (width 0.25) (layer "F.Cu") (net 17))
 (segment (start 192.734 109.6116) (end 186.234 109.6116) (width 0.25) (layer "F.Cu") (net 17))
 (segment (start 170.8404 85.0392) (end 169.0116 83.2104) (width 0.25) (layer "F.Cu") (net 17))
 (segment (start 186.234 103.1252) (end 178.7652 95.6564) (width 0.25) (layer "F.Cu") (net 17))
 (via (at 170.8404 93.7768) (size 0.8) (drill 0.4) (layers "F.Cu" "B.Cu") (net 17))
 (via (at 178.7652 95.6564) (size 0.8) (drill 0.4) (layers "F.Cu" "B.Cu") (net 17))
 (segment (start 178.7652 95.6564) (end 172.72 95.6564) (width 0.25) (layer "B.Cu") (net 17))
 (segment (start 172.72 95.6564) (end 170.8404 93.7768) (width 0.25) (layer "B.Cu") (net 17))
 (segment (start 178.9684 86.868) (end 175.0568 82.9564) (width 0.25) (layer "F.Cu") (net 4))
 (segment (start 175.0568 82.9564) (end 175.0568 69.1896) (width 0.25) (layer "F.Cu") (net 4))
 (segment (start 183.896 93.0656) (end 178.9684 93.0656) (width 0.25) (layer "F.Cu") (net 4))
 (segment (start 198.7308 107.9004) (end 183.896 93.0656) (width 0.25) (layer "F.Cu") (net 4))
 (segment (start 198.7308 109.6624) (end 198.7308 107.9004) (width 0.25) (layer "F.Cu") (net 4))
 (segment (start 205.2308 109.6624) (end 198.7308 109.6624) (width 0.25) (layer "F.Cu") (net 4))
 (segment (start 175.0568 69.1896) (end 174.2948 68.4276) (width 0.25) (layer "F.Cu") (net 4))
 (segment (start 178.9684 93.0656) (end 178.9684 86.868) (width 0.25) (layer "F.Cu") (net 4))
 (segment (start 132.9834 50.6649) (end 137.4821 50.6649) (width 0.25) (layer "F.Cu") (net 19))
 (segment (start 166.3192 66.2432) (end 166.6748 65.8876) (width 0.25) (layer "F.Cu") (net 19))
 (segment (start 157.3784 68.4784) (end 158.533 68.4784) (width 0.25) (layer "F.Cu") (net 19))
 (segment (start 158.533 68.4784) (end 160.2094 66.802) (width 0.25) (layer "F.Cu") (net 19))
 (segment (start 162.6616 66.2432) (end 166.3192 66.2432) (width 0.25) (layer "F.Cu") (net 19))
 (segment (start 137.4821 50.6649) (end 145.3896 58.5724) (width 0.25) (layer "F.Cu") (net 19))
 (via (at 145.3896 58.5724) (size 0.8) (drill 0.4) (layers "F.Cu" "B.Cu") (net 19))
 (via (at 160.2094 66.802) (size 0.8) (drill 0.4) (layers "F.Cu" "B.Cu") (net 19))
 (via (at 162.6616 66.2432) (size 0.8) (drill 0.4) (layers "F.Cu" "B.Cu") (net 19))
 (via (at 157.3784 68.4784) (size 0.8) (drill 0.4) (layers "F.Cu" "B.Cu") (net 19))
 (segment (start 160.2094 66.802) (end 162.1028 66.802) (width 0.25) (layer "B.Cu") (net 19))
 (segment (start 145.3896 67.564) (end 146.1008 68.2752) (width 0.25) (layer "B.Cu") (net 19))
 (segment (start 145.3896 58.5724) (end 145.3896 67.564) (width 0.25) (layer "B.Cu") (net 19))
 (segment (start 162.1028 66.802) (end 162.6616 66.2432) (width 0.25) (layer "B.Cu") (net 19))
 (segment (start 157.1752 68.2752) (end 157.3784 68.4784) (width 0.25) (layer "B.Cu") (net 19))
 (segment (start 146.1008 68.2752) (end 157.1752 68.2752) (width 0.25) (layer "B.Cu") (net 19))
 (segment (start 187.6044 55.7784) (end 181.9656 55.7784) (width 0.25) (layer "F.Cu") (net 12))
 (segment (start 197.2564 52.1716) (end 196.3928 52.1716) (width 0.25) (layer "F.Cu") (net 12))
 (segment (start 182.2196 56.0324) (end 181.9148 55.7276) (width 0.25) (layer "F.Cu") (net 12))
 (segment (start 220.5453 48.9712) (end 213.106 48.9712) (width 0.25) (layer "F.Cu") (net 12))
 (segment (start 221.9342 50.3601) (end 220.5453 48.9712) (width 0.25) (layer "F.Cu") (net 12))
 (segment (start 181.9656 55.7784) (end 181.9148 55.7276) (width 0.25) (layer "F.Cu") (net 12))
 (segment (start 196.3928 52.1716) (end 193.4464 55.118) (width 0.25) (layer "F.Cu") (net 12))
 (via (at 187.6044 55.7784) (size 0.8) (drill 0.4) (layers "F.Cu" "B.Cu") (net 12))
 (via (at 193.4464 55.118) (size 0.8) (drill 0.4) (layers "F.Cu" "B.Cu") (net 12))
 (via (at 213.106 48.9712) (size 0.8) (drill 0.4) (layers "F.Cu" "B.Cu") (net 12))
 (via (at 197.2564 52.1716) (size 0.8) (drill 0.4) (layers "F.Cu" "B.Cu") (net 12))
 (segment (start 193.4464 55.118) (end 188.2648 55.118) (width 0.25) (layer "B.Cu") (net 12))
 (segment (start 188.2648 55.118) (end 187.6044 55.7784) (width 0.25) (layer "B.Cu") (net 12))
 (segment (start 213.106 48.9712) (end 210.603 51.4742) (width 0.25) (layer "B.Cu") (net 12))
 (segment (start 197.9538 51.4742) (end 197.2564 52.1716) (width 0.25) (layer "B.Cu") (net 12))
 (segment (start 210.603 51.4742) (end 197.9538 51.4742) (width 0.25) (layer "B.Cu") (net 12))
 (segment (start 183.642 89.5604) (end 182.2704 89.5604) (width 0.25) (layer "F.Cu") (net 7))
 (segment (start 176.8348 76.5048) (end 176.8348 68.4276) (width 0.25) (layer "F.Cu") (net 7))
 (segment (start 193.4972 99.4156) (end 183.642 89.5604) (width 0.25) (layer "F.Cu") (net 7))
 (segment (start 209.296 99.4156) (end 193.4972 99.4156) (width 0.25) (layer "F.Cu") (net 7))
 (segment (start 182.2704 81.9404) (end 176.8348 76.5048) (width 0.25) (layer "F.Cu") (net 7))
 (segment (start 211.0752 109.7132) (end 209.296 107.934) (width 0.25) (layer "F.Cu") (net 7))
 (segment (start 209.296 107.934) (end 209.296 99.4156) (width 0.25) (layer "F.Cu") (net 7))
 (segment (start 182.2704 89.5604) (end 182.2704 81.9404) (width 0.25) (layer "F.Cu") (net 7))
 (segment (start 217.5752 109.7132) (end 211.0752 109.7132) (width 0.25) (layer "F.Cu") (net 7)))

